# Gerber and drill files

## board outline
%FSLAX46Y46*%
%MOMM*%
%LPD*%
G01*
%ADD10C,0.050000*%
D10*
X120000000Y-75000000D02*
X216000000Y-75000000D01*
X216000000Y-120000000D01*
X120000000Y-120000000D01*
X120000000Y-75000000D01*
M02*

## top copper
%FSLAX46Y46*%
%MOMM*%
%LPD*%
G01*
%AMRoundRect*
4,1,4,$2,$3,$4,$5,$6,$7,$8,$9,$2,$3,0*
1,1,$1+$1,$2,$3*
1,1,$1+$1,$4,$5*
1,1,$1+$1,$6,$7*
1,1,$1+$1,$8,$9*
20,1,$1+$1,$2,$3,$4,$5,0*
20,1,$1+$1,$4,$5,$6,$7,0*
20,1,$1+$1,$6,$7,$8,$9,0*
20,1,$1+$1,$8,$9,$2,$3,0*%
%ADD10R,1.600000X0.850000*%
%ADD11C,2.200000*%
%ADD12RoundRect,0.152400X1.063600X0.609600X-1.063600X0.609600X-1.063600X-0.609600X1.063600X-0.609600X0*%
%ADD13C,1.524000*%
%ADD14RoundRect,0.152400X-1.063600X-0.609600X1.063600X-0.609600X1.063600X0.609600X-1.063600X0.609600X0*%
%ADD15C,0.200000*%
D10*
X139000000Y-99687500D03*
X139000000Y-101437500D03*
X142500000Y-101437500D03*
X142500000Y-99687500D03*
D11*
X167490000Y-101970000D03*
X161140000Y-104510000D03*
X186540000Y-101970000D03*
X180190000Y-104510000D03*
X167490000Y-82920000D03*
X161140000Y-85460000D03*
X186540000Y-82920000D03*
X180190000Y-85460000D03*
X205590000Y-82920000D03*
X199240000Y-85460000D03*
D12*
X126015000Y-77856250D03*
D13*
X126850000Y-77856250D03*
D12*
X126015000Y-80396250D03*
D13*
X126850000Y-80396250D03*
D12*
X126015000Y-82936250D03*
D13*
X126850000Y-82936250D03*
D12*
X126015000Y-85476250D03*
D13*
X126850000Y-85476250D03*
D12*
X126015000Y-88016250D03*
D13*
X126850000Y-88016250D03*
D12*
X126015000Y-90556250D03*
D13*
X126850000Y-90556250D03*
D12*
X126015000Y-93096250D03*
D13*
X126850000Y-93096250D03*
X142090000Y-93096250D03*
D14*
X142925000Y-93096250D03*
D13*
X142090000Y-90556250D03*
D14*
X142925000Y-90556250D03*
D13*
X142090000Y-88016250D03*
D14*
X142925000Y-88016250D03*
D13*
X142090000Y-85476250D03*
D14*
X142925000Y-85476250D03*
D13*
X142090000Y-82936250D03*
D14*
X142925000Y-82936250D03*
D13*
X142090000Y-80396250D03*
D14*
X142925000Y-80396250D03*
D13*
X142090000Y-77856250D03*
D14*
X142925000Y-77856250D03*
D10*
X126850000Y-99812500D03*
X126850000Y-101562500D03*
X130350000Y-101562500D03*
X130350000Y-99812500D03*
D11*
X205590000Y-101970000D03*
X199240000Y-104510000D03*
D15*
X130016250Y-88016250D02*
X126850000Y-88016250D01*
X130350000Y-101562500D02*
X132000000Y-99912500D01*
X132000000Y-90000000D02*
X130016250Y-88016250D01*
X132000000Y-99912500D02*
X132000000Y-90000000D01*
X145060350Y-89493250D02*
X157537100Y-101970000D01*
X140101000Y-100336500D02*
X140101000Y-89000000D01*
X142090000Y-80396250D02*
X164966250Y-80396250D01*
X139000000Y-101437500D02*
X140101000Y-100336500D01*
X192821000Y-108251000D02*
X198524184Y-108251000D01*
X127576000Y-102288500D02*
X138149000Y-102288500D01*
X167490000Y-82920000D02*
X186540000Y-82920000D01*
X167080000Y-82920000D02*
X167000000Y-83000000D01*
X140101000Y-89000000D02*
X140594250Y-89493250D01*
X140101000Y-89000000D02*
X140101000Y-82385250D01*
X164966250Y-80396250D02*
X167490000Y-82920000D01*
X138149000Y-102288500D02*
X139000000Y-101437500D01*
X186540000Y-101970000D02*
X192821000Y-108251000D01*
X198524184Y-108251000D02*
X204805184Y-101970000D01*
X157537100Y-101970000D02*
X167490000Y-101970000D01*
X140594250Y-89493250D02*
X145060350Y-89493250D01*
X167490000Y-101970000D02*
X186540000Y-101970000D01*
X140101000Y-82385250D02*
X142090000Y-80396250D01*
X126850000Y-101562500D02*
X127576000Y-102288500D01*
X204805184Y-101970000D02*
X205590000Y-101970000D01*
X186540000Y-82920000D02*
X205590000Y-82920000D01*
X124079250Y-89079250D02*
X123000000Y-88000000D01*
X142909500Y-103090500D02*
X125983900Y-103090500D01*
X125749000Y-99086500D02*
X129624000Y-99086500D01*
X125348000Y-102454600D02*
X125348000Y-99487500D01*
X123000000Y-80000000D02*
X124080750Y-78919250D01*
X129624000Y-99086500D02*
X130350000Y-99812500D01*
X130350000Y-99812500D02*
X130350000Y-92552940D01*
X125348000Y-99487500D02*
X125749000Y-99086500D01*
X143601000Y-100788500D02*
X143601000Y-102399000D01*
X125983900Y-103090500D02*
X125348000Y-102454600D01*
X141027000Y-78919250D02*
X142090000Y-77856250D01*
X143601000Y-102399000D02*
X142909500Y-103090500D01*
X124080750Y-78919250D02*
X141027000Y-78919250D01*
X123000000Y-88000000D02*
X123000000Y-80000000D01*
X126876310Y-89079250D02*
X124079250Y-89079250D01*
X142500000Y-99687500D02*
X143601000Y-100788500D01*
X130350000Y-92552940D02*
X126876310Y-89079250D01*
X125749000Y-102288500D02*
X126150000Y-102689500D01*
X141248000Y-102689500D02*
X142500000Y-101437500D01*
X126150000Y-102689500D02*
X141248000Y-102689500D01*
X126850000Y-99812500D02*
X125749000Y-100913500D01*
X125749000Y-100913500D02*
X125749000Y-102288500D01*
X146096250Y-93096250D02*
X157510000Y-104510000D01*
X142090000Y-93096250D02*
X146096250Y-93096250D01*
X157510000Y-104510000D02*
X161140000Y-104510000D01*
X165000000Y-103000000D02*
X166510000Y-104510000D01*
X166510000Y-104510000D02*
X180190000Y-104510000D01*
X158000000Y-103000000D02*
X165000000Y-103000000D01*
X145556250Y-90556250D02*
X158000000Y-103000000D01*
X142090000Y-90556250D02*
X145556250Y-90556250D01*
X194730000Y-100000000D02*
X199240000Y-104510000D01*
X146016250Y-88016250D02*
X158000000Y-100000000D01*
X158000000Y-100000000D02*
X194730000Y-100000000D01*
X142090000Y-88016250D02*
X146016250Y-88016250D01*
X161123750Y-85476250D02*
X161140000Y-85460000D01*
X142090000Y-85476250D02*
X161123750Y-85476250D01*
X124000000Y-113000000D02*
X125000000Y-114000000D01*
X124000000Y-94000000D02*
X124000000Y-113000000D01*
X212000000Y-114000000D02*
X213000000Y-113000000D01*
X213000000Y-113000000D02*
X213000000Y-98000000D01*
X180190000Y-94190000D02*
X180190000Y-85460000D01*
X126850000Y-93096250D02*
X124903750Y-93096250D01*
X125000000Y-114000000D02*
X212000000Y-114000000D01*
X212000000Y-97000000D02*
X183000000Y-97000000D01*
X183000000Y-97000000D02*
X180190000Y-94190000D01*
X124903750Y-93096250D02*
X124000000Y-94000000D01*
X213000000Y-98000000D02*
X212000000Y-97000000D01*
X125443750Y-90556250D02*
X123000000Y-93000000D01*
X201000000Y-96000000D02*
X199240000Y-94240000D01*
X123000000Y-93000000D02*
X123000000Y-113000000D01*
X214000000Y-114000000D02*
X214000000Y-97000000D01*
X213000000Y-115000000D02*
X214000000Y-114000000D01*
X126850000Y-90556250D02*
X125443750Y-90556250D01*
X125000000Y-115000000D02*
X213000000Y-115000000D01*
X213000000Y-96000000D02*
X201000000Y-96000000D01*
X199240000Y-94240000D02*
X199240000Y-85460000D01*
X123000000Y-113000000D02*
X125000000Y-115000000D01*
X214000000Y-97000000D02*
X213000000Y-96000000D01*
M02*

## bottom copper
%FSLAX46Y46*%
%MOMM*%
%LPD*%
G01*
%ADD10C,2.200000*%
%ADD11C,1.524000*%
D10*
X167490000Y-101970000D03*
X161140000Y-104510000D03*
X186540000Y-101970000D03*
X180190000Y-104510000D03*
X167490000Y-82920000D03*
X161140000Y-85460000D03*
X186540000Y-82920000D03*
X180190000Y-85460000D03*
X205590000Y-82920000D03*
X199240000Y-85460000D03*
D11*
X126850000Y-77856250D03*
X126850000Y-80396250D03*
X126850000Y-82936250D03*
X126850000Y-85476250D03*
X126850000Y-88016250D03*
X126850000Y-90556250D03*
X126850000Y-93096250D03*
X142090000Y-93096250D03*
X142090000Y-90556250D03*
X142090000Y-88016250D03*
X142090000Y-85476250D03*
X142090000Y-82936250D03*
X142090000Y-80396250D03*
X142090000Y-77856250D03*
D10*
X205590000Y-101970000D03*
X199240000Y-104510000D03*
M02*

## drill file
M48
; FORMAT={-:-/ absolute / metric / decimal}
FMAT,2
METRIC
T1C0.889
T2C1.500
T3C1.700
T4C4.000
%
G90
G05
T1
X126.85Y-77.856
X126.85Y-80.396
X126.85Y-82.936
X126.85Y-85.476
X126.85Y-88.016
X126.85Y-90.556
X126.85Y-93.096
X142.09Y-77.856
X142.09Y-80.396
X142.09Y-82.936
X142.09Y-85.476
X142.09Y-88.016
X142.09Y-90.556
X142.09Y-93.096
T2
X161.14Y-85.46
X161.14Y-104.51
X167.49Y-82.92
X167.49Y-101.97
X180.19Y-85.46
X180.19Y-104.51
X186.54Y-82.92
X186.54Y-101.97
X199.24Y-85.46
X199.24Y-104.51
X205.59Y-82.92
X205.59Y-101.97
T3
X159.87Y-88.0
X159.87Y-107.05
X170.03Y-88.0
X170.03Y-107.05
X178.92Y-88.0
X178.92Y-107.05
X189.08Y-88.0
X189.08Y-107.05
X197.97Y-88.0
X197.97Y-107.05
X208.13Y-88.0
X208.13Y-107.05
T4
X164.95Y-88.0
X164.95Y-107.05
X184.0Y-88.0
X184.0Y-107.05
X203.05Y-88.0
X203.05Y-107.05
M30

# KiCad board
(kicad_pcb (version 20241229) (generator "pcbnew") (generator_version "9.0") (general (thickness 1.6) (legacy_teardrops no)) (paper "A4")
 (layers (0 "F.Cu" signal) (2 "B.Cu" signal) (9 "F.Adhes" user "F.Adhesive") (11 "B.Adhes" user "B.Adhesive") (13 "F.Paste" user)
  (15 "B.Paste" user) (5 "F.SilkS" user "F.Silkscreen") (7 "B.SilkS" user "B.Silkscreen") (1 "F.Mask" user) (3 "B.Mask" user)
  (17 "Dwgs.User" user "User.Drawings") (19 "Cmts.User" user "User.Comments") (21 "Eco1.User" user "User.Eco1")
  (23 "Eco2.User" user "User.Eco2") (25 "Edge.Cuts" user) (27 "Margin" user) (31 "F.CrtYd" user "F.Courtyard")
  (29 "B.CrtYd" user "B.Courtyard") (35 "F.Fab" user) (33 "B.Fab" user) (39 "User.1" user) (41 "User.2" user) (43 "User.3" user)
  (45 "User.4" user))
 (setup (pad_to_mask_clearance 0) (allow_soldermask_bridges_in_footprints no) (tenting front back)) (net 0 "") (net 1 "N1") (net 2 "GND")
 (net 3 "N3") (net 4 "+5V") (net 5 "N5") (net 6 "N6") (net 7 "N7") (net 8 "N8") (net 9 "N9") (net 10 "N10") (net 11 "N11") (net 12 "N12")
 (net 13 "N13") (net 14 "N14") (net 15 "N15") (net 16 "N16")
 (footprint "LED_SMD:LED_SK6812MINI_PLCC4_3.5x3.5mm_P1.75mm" (layer "F.Cu") (at 140.75 100.5625)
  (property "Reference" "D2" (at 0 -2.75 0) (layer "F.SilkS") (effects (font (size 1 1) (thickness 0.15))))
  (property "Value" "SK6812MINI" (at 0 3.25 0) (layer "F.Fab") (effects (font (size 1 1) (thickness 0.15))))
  (pad "1" smd rect (at -1.75 -0.875) (size 1.6 0.85) (layers "F.Cu" "F.Mask" "F.Paste") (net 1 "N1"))
  (pad "2" smd rect (at -1.75 0.875) (size 1.6 0.85) (layers "F.Cu" "F.Mask" "F.Paste") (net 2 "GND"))
  (pad "3" smd rect (at 1.75 0.875) (size 1.6 0.85) (layers "F.Cu" "F.Mask" "F.Paste") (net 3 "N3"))
  (pad "4" smd rect (at 1.75 -0.875) (size 1.6 0.85) (layers "F.Cu" "F.Mask" "F.Paste") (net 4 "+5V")))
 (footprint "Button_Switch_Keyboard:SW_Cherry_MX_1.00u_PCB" (layer "F.Cu") (at 167.49 101.97)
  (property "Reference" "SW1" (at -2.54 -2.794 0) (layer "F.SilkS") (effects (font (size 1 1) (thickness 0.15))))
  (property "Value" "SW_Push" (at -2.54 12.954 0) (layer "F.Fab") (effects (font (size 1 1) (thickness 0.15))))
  (pad "" np_thru_hole circle (at -7.62 5.08) (size 1.7 1.7) (drill 1.7) (layers "*.Cu" "*.Mask"))
  (pad "" np_thru_hole circle (at -2.54 5.08) (size 4 4) (drill 4) (layers "*.Cu" "*.Mask"))
  (pad "" np_thru_hole circle (at 2.54 5.08) (size 1.7 1.7) (drill 1.7) (layers "*.Cu" "*.Mask"))
  (pad "1" thru_hole circle (at 0 0) (size 2.2 2.2) (drill 1.5) (layers "*.Cu" "*.Mask") (remove_unused_layers no) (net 2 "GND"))
  (pad "2" thru_hole circle (at -6.35 2.54) (size 2.2 2.2) (drill 1.5) (layers "*.Cu" "*.Mask") (remove_unused_layers no) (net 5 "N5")))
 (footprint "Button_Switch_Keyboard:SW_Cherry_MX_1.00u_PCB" (layer "F.Cu") (at 186.54 101.97)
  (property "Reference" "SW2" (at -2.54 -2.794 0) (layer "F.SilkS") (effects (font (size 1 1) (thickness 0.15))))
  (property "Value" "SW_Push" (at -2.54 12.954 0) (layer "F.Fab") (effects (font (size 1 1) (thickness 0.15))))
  (pad "" np_thru_hole circle (at -7.62 5.08) (size 1.7 1.7) (drill 1.7) (layers "*.Cu" "*.Mask"))
  (pad "" np_thru_hole circle (at -2.54 5.08) (size 4 4) (drill 4) (layers "*.Cu" "*.Mask"))
  (pad "" np_thru_hole circle (at 2.54 5.08) (size 1.7 1.7) (drill 1.7) (layers "*.Cu" "*.Mask"))
  (pad "1" thru_hole circle (at 0 0) (size 2.2 2.2) (drill 1.5) (layers "*.Cu" "*.Mask") (remove_unused_layers no) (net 2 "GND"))
  (pad "2" thru_hole circle (at -6.35 2.54) (size 2.2 2.2) (drill 1.5) (layers "*.Cu" "*.Mask") (remove_unused_layers no) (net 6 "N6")))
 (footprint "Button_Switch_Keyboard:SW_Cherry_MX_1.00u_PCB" (layer "F.Cu") (at 167.49 82.92)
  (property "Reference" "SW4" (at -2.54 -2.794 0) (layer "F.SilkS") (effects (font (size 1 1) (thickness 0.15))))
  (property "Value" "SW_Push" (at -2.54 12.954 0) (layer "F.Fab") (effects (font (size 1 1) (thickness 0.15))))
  (pad "" np_thru_hole circle (at -7.62 5.08) (size 1.7 1.7) (drill 1.7) (layers "*.Cu" "*.Mask"))
  (pad "" np_thru_hole circle (at -2.54 5.08) (size 4 4) (drill 4) (layers "*.Cu" "*.Mask"))
  (pad "" np_thru_hole circle (at 2.54 5.08) (size 1.7 1.7) (drill 1.7) (layers "*.Cu" "*.Mask"))
  (pad "1" thru_hole circle (at 0 0) (size 2.2 2.2) (drill 1.5) (layers "*.Cu" "*.Mask") (remove_unused_layers no) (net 2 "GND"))
  (pad "2" thru_hole circle (at -6.35 2.54) (size 2.2 2.2) (drill 1.5) (layers "*.Cu" "*.Mask") (remove_unused_layers no) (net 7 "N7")))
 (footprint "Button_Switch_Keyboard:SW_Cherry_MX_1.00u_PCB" (layer "F.Cu") (at 186.54 82.92)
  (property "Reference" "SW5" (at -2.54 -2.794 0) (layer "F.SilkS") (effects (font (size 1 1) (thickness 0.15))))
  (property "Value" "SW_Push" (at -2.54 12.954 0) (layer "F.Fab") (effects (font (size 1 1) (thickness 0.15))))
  (pad "" np_thru_hole circle (at -7.62 5.08) (size 1.7 1.7) (drill 1.7) (layers "*.Cu" "*.Mask"))
  (pad "" np_thru_hole circle (at -2.54 5.08) (size 4 4) (drill 4) (layers "*.Cu" "*.Mask"))
  (pad "" np_thru_hole circle (at 2.54 5.08) (size 1.7 1.7) (drill 1.7) (layers "*.Cu" "*.Mask"))
  (pad "1" thru_hole circle (at 0 0) (size 2.2 2.2) (drill 1.5) (layers "*.Cu" "*.Mask") (remove_unused_layers no) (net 2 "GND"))
  (pad "2" thru_hole circle (at -6.35 2.54) (size 2.2 2.2) (drill 1.5) (layers "*.Cu" "*.Mask") (remove_unused_layers no) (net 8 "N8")))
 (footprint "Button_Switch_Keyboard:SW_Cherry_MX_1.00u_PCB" (layer "F.Cu") (at 205.59 82.92)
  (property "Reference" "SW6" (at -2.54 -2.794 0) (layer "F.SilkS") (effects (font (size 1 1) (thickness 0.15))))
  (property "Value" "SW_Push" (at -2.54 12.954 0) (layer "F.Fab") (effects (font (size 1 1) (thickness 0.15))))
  (pad "" np_thru_hole circle (at -7.62 5.08) (size 1.7 1.7) (drill 1.7) (layers "*.Cu" "*.Mask"))
  (pad "" np_thru_hole circle (at -2.54 5.08) (size 4 4) (drill 4) (layers "*.Cu" "*.Mask"))
  (pad "" np_thru_hole circle (at 2.54 5.08) (size 1.7 1.7) (drill 1.7) (layers "*.Cu" "*.Mask"))
  (pad "1" thru_hole circle (at 0 0) (size 2.2 2.2) (drill 1.5) (layers "*.Cu" "*.Mask") (remove_unused_layers no) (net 2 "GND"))
  (pad "2" thru_hole circle (at -6.35 2.54) (size 2.2 2.2) (drill 1.5) (layers "*.Cu" "*.Mask") (remove_unused_layers no) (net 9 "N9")))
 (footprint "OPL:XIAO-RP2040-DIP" (layer "F.Cu") (at 134.47 85.47625)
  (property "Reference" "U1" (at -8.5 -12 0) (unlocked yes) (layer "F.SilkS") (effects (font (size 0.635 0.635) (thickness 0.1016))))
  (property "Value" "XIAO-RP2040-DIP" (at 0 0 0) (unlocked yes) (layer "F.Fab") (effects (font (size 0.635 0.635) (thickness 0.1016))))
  (pad "1" smd roundrect (at -8.455 -7.62 180) (size 2.432 1.524) (layers "F.Cu" "F.Mask") (roundrect_rratio 0.1) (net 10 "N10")
   (thermal_bridge_angle 45))
  (pad "1" thru_hole circle (at -7.62 -7.62 180) (size 1.524 1.524) (drill 0.889) (layers "*.Cu" "*.Mask") (remove_unused_layers no)
   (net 10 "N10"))
  (pad "2" smd roundrect (at -8.455 -5.08 180) (size 2.432 1.524) (layers "F.Cu" "F.Mask") (roundrect_rratio 0.1) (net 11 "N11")
   (thermal_bridge_angle 45))
  (pad "2" thru_hole circle (at -7.62 -5.08 180) (size 1.524 1.524) (drill 0.889) (layers "*.Cu" "*.Mask") (remove_unused_layers no)
   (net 11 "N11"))
  (pad "3" smd roundrect (at -8.455 -2.54 180) (size 2.432 1.524) (layers "F.Cu" "F.Mask") (roundrect_rratio 0.1) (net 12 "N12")
   (thermal_bridge_angle 45))
  (pad "3" thru_hole circle (at -7.62 -2.54 180) (size 1.524 1.524) (drill 0.889) (layers "*.Cu" "*.Mask") (remove_unused_layers no)
   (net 12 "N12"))
  (pad "4" smd roundrect (at -8.455 0 180) (size 2.432 1.524) (layers "F.Cu" "F.Mask") (roundrect_rratio 0.1) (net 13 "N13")
   (thermal_bridge_angle 45))
  (pad "4" thru_hole circle (at -7.62 0 180) (size 1.524 1.524) (drill 0.889) (layers "*.Cu" "*.Mask") (remove_unused_layers no)
   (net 13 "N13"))
  (pad "5" smd roundrect (at -8.455 2.54 180) (size 2.432 1.524) (layers "F.Cu" "F.Mask") (roundrect_rratio 0.1) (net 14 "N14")
   (thermal_bridge_angle 45))
  (pad "5" thru_hole circle (at -7.62 2.54 180) (size 1.524 1.524) (drill 0.889) (layers "*.Cu" "*.Mask") (remove_unused_layers no)
   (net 14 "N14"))
  (pad "6" smd roundrect (at -8.455 5.08 180) (size 2.432 1.524) (layers "F.Cu" "F.Mask") (roundrect_rratio 0.1) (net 9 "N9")
   (thermal_bridge_angle 45))
  (pad "6" thru_hole circle (at -7.62 5.08 180) (size 1.524 1.524) (drill 0.889) (layers "*.Cu" "*.Mask") (remove_unused_layers no)
   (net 9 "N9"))
  (pad "7" smd roundrect (at -8.455 7.62 180) (size 2.432 1.524) (layers "F.Cu" "F.Mask") (roundrect_rratio 0.1) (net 8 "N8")
   (thermal_bridge_angle 45))
  (pad "7" thru_hole circle (at -7.62 7.62 180) (size 1.524 1.524) (drill 0.889) (layers "*.Cu" "*.Mask") (remove_unused_layers no)
   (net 8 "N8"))
  (pad "8" thru_hole circle (at 7.62 7.62) (size 1.524 1.524) (drill 0.889) (layers "*.Cu" "*.Mask") (remove_unused_layers no) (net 5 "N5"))
  (pad "8" smd roundrect (at 8.455 7.62) (size 2.432 1.524) (layers "F.Cu" "F.Mask") (roundrect_rratio 0.1) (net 5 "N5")
   (thermal_bridge_angle 45))
  (pad "9" thru_hole circle (at 7.62 5.08) (size 1.524 1.524) (drill 0.889) (layers "*.Cu" "*.Mask") (remove_unused_layers no) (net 6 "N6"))
  (pad "9" smd roundrect (at 8.455 5.08) (size 2.432 1.524) (layers "F.Cu" "F.Mask") (roundrect_rratio 0.1) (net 6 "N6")
   (thermal_bridge_angle 45))
  (pad "10" thru_hole circle (at 7.62 2.54) (size 1.524 1.524) (drill 0.889) (layers "*.Cu" "*.Mask") (remove_unused_layers no)
   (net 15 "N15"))
  (pad "10" smd roundrect (at 8.455 2.54) (size 2.432 1.524) (layers "F.Cu" "F.Mask") (roundrect_rratio 0.1) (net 15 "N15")
   (thermal_bridge_angle 45))
  (pad "11" thru_hole circle (at 7.62 0) (size 1.524 1.524) (drill 0.889) (layers "*.Cu" "*.Mask") (remove_unused_layers no) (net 7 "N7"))
  (pad "11" smd roundrect (at 8.455 0) (size 2.432 1.524) (layers "F.Cu" "F.Mask") (roundrect_rratio 0.1) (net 7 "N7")
   (thermal_bridge_angle 45))
  (pad "12" thru_hole circle (at 7.62 -2.54) (size 1.524 1.524) (drill 0.889) (layers "*.Cu" "*.Mask") (remove_unused_layers no)
   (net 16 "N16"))
  (pad "12" smd roundrect (at 8.455 -2.54) (size 2.432 1.524) (layers "F.Cu" "F.Mask") (roundrect_rratio 0.1) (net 16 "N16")
   (thermal_bridge_angle 45))
  (pad "13" thru_hole circle (at 7.62 -5.08) (size 1.524 1.524) (drill 0.889) (layers "*.Cu" "*.Mask") (remove_unused_layers no)
   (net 2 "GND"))
  (pad "13" smd roundrect (at 8.455 -5.08) (size 2.432 1.524) (layers "F.Cu" "F.Mask") (roundrect_rratio 0.1) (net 2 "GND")
   (thermal_bridge_angle 45))
  (pad "14" thru_hole circle (at 7.62 -7.62) (size 1.524 1.524) (drill 0.889) (layers "*.Cu" "*.Mask") (remove_unused_layers no)
   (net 4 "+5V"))
  (pad "14" smd roundrect (at 8.455 -7.62) (size 2.432 1.524) (layers "F.Cu" "F.Mask") (roundrect_rratio 0.1) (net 4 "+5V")
   (thermal_bridge_angle 45)))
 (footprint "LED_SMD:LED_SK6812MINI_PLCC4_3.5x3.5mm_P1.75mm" (layer "F.Cu") (at 128.6 100.6875)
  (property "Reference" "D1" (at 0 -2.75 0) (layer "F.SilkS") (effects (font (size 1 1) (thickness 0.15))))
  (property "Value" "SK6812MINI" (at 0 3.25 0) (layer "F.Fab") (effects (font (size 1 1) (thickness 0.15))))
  (pad "1" smd rect (at -1.75 -0.875) (size 1.6 0.85) (layers "F.Cu" "F.Mask" "F.Paste") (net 3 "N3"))
  (pad "2" smd rect (at -1.75 0.875) (size 1.6 0.85) (layers "F.Cu" "F.Mask" "F.Paste") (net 2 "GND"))
  (pad "3" smd rect (at 1.75 0.875) (size 1.6 0.85) (layers "F.Cu" "F.Mask" "F.Paste") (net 14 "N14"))
  (pad "4" smd rect (at 1.75 -0.875) (size 1.6 0.85) (layers "F.Cu" "F.Mask" "F.Paste") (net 4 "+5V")))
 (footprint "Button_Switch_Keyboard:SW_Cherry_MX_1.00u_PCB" (layer "F.Cu") (at 205.59 101.97)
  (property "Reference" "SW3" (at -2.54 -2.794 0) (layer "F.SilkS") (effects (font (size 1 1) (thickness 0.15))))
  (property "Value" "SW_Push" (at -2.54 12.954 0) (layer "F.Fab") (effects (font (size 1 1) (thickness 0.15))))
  (pad "" np_thru_hole circle (at -7.62 5.08) (size 1.7 1.7) (drill 1.7) (layers "*.Cu" "*.Mask"))
  (pad "" np_thru_hole circle (at -2.54 5.08) (size 4 4) (drill 4) (layers "*.Cu" "*.Mask"))
  (pad "" np_thru_hole circle (at 2.54 5.08) (size 1.7 1.7) (drill 1.7) (layers "*.Cu" "*.Mask"))
  (pad "1" thru_hole circle (at 0 0) (size 2.2 2.2) (drill 1.5) (layers "*.Cu" "*.Mask") (remove_unused_layers no) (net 2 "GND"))
  (pad "2" thru_hole circle (at -6.35 2.54) (size 2.2 2.2) (drill 1.5) (layers "*.Cu" "*.Mask") (remove_unused_layers no) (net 15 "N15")))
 (gr_rect (start 120 75) (end 216 120) (stroke (width 0.05) (type default)) (fill no) (layer "Edge.Cuts"))
 (segment (start 130.01625 88.01625) (end 126.85 88.01625) (width 0.2) (layer "F.Cu") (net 14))
 (segment (start 130.35 101.5625) (end 132 99.9125) (width 0.2) (layer "F.Cu") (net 14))
 (segment (start 132 90) (end 130.01625 88.01625) (width 0.2) (layer "F.Cu") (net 14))
 (segment (start 132 99.9125) (end 132 90) (width 0.2) (layer "F.Cu") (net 14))
 (segment (start 145.06035 89.49325) (end 157.5371 101.97) (width 0.2) (layer "F.Cu") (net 2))
 (segment (start 140.101 100.3365) (end 140.101 89) (width 0.2) (layer "F.Cu") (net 2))
 (segment (start 142.09 80.39625) (end 164.96625 80.39625) (width 0.2) (layer "F.Cu") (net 2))
 (segment (start 139 101.4375) (end 140.101 100.3365) (width 0.2) (layer "F.Cu") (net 2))
 (segment (start 192.821 108.251) (end 198.524184 108.251) (width 0.2) (layer "F.Cu") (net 2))
 (segment (start 127.576 102.2885) (end 138.149 102.2885) (width 0.2) (layer "F.Cu") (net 2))
 (segment (start 167.49 82.92) (end 186.54 82.92) (width 0.2) (layer "F.Cu") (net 2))
 (segment (start 167.08 82.92) (end 167 83) (width 0.2) (layer "F.Cu") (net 2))
 (segment (start 140.101 89) (end 140.59425 89.49325) (width 0.2) (layer "F.Cu") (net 2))
 (segment (start 140.101 89) (end 140.101 82.38525) (width 0.2) (layer "F.Cu") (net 2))
 (segment (start 164.96625 80.39625) (end 167.49 82.92) (width 0.2) (layer "F.Cu") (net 2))
 (segment (start 138.149 102.2885) (end 139 101.4375) (width 0.2) (layer "F.Cu") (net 2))
 (segment (start 186.54 101.97) (end 192.821 108.251) (width 0.2) (layer "F.Cu") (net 2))
 (segment (start 198.524184 108.251) (end 204.805184 101.97) (width 0.2) (layer "F.Cu") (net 2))
 (segment (start 157.5371 101.97) (end 167.49 101.97) (width 0.2) (layer "F.Cu") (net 2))
 (segment (start 140.59425 89.49325) (end 145.06035 89.49325) (width 0.2) (layer "F.Cu") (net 2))
 (segment (start 167.49 101.97) (end 186.54 101.97) (width 0.2) (layer "F.Cu") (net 2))
 (segment (start 140.101 82.38525) (end 142.09 80.39625) (width 0.2) (layer "F.Cu") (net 2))
 (segment (start 126.85 101.5625) (end 127.576 102.2885) (width 0.2) (layer "F.Cu") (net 2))
 (segment (start 204.805184 101.97) (end 205.59 101.97) (width 0.2) (layer "F.Cu") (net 2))
 (segment (start 186.54 82.92) (end 205.59 82.92) (width 0.2) (layer "F.Cu") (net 2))
 (segment (start 124.07925 89.07925) (end 123 88) (width 0.2) (layer "F.Cu") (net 4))
 (segment (start 142.9095 103.0905) (end 125.9839 103.0905) (width 0.2) (layer "F.Cu") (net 4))
 (segment (start 125.749 99.0865) (end 129.624 99.0865) (width 0.2) (layer "F.Cu") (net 4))
 (segment (start 125.348 102.4546) (end 125.348 99.4875) (width 0.2) (layer "F.Cu") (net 4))
 (segment (start 123 80) (end 124.08075 78.91925) (width 0.2) (layer "F.Cu") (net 4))
 (segment (start 129.624 99.0865) (end 130.35 99.8125) (width 0.2) (layer "F.Cu") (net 4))
 (segment (start 130.35 99.8125) (end 130.35 92.55294) (width 0.2) (layer "F.Cu") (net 4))
 (segment (start 125.348 99.4875) (end 125.749 99.0865) (width 0.2) (layer "F.Cu") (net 4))
 (segment (start 143.601 100.7885) (end 143.601 102.399) (width 0.2) (layer "F.Cu") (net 4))
 (segment (start 125.9839 103.0905) (end 125.348 102.4546) (width 0.2) (layer "F.Cu") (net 4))
 (segment (start 141.027 78.91925) (end 142.09 77.85625) (width 0.2) (layer "F.Cu") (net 4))
 (segment (start 143.601 102.399) (end 142.9095 103.0905) (width 0.2) (layer "F.Cu") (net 4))
 (segment (start 124.08075 78.91925) (end 141.027 78.91925) (width 0.2) (layer "F.Cu") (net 4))
 (segment (start 123 88) (end 123 80) (width 0.2) (layer "F.Cu") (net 4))
 (segment (start 126.87631 89.07925) (end 124.07925 89.07925) (width 0.2) (layer "F.Cu") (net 4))
 (segment (start 142.5 99.6875) (end 143.601 100.7885) (width 0.2) (layer "F.Cu") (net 4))
 (segment (start 130.35 92.55294) (end 126.87631 89.07925) (width 0.2) (layer "F.Cu") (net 4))
 (segment (start 125.749 102.2885) (end 126.15 102.6895) (width 0.2) (layer "F.Cu") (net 3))
 (segment (start 141.248 102.6895) (end 142.5 101.4375) (width 0.2) (layer "F.Cu") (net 3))
 (segment (start 126.15 102.6895) (end 141.248 102.6895) (width 0.2) (layer "F.Cu") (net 3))
 (segment (start 126.85 99.8125) (end 125.749 100.9135) (width 0.2) (layer "F.Cu") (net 3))
 (segment (start 125.749 100.9135) (end 125.749 102.2885) (width 0.2) (layer "F.Cu") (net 3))
 (segment (start 146.09625 93.09625) (end 157.51 104.51) (width 0.2) (layer "F.Cu") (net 5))
 (segment (start 142.09 93.09625) (end 146.09625 93.09625) (width 0.2) (layer "F.Cu") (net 5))
 (segment (start 157.51 104.51) (end 161.14 104.51) (width 0.2) (layer "F.Cu") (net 5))
 (segment (start 165 103) (end 166.51 104.51) (width 0.2) (layer "F.Cu") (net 6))
 (segment (start 166.51 104.51) (end 180.19 104.51) (width 0.2) (layer "F.Cu") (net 6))
 (segment (start 158 103) (end 165 103) (width 0.2) (layer "F.Cu") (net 6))
 (segment (start 145.55625 90.55625) (end 158 103) (width 0.2) (layer "F.Cu") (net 6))
 (segment (start 142.09 90.55625) (end 145.55625 90.55625) (width 0.2) (layer "F.Cu") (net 6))
 (segment (start 194.73 100) (end 199.24 104.51) (width 0.2) (layer "F.Cu") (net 15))
 (segment (start 146.01625 88.01625) (end 158 100) (width 0.2) (layer "F.Cu") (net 15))
 (segment (start 158 100) (end 194.73 100) (width 0.2) (layer "F.Cu") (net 15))
 (segment (start 142.09 88.01625) (end 146.01625 88.01625) (width 0.2) (layer "F.Cu") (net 15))
 (segment (start 161.12375 85.47625) (end 161.14 85.46) (width 0.2) (layer "F.Cu") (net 7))
 (segment (start 142.09 85.47625) (end 161.12375 85.47625) (width 0.2) (layer "F.Cu") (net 7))
 (segment (start 124 113) (end 125 114) (width 0.2) (layer "F.Cu") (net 8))
 (segment (start 124 94) (end 124 113) (width 0.2) (layer "F.Cu") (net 8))
 (segment (start 212 114) (end 213 113) (width 0.2) (layer "F.Cu") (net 8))
 (segment (start 213 113) (end 213 98) (width 0.2) (layer "F.Cu") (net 8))
 (segment (start 180.19 94.19) (end 180.19 85.46) (width 0.2) (layer "F.Cu") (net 8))
 (segment (start 126.85 93.09625) (end 124.90375 93.09625) (width 0.2) (layer "F.Cu") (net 8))
 (segment (start 125 114) (end 212 114) (width 0.2) (layer "F.Cu") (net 8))
 (segment (start 212 97) (end 183 97) (width 0.2) (layer "F.Cu") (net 8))
 (segment (start 183 97) (end 180.19 94.19) (width 0.2) (layer "F.Cu") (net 8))
 (segment (start 124.90375 93.09625) (end 124 94) (width 0.2) (layer "F.Cu") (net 8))
 (segment (start 213 98) (end 212 97) (width 0.2) (layer "F.Cu") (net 8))
 (segment (start 125.44375 90.55625) (end 123 93) (width 0.2) (layer "F.Cu") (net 9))
 (segment (start 201 96) (end 199.24 94.24) (width 0.2) (layer "F.Cu") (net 9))
 (segment (start 123 93) (end 123 113) (width 0.2) (layer "F.Cu") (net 9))
 (segment (start 214 114) (end 214 97) (width 0.2) (layer "F.Cu") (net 9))
 (segment (start 213 115) (end 214 114) (width 0.2) (layer "F.Cu") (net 9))
 (segment (start 126.85 90.55625) (end 125.44375 90.55625) (width 0.2) (layer "F.Cu") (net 9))
 (segment (start 125 115) (end 213 115) (width 0.2) (layer "F.Cu") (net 9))
 (segment (start 213 96) (end 201 96) (width 0.2) (layer "F.Cu") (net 9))
 (segment (start 199.24 94.24) (end 199.24 85.46) (width 0.2) (layer "F.Cu") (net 9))
 (segment (start 123 113) (end 125 115) (width 0.2) (layer "F.Cu") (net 9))
 (segment (start 214 97) (end 213 96) (width 0.2) (layer "F.Cu") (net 9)))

